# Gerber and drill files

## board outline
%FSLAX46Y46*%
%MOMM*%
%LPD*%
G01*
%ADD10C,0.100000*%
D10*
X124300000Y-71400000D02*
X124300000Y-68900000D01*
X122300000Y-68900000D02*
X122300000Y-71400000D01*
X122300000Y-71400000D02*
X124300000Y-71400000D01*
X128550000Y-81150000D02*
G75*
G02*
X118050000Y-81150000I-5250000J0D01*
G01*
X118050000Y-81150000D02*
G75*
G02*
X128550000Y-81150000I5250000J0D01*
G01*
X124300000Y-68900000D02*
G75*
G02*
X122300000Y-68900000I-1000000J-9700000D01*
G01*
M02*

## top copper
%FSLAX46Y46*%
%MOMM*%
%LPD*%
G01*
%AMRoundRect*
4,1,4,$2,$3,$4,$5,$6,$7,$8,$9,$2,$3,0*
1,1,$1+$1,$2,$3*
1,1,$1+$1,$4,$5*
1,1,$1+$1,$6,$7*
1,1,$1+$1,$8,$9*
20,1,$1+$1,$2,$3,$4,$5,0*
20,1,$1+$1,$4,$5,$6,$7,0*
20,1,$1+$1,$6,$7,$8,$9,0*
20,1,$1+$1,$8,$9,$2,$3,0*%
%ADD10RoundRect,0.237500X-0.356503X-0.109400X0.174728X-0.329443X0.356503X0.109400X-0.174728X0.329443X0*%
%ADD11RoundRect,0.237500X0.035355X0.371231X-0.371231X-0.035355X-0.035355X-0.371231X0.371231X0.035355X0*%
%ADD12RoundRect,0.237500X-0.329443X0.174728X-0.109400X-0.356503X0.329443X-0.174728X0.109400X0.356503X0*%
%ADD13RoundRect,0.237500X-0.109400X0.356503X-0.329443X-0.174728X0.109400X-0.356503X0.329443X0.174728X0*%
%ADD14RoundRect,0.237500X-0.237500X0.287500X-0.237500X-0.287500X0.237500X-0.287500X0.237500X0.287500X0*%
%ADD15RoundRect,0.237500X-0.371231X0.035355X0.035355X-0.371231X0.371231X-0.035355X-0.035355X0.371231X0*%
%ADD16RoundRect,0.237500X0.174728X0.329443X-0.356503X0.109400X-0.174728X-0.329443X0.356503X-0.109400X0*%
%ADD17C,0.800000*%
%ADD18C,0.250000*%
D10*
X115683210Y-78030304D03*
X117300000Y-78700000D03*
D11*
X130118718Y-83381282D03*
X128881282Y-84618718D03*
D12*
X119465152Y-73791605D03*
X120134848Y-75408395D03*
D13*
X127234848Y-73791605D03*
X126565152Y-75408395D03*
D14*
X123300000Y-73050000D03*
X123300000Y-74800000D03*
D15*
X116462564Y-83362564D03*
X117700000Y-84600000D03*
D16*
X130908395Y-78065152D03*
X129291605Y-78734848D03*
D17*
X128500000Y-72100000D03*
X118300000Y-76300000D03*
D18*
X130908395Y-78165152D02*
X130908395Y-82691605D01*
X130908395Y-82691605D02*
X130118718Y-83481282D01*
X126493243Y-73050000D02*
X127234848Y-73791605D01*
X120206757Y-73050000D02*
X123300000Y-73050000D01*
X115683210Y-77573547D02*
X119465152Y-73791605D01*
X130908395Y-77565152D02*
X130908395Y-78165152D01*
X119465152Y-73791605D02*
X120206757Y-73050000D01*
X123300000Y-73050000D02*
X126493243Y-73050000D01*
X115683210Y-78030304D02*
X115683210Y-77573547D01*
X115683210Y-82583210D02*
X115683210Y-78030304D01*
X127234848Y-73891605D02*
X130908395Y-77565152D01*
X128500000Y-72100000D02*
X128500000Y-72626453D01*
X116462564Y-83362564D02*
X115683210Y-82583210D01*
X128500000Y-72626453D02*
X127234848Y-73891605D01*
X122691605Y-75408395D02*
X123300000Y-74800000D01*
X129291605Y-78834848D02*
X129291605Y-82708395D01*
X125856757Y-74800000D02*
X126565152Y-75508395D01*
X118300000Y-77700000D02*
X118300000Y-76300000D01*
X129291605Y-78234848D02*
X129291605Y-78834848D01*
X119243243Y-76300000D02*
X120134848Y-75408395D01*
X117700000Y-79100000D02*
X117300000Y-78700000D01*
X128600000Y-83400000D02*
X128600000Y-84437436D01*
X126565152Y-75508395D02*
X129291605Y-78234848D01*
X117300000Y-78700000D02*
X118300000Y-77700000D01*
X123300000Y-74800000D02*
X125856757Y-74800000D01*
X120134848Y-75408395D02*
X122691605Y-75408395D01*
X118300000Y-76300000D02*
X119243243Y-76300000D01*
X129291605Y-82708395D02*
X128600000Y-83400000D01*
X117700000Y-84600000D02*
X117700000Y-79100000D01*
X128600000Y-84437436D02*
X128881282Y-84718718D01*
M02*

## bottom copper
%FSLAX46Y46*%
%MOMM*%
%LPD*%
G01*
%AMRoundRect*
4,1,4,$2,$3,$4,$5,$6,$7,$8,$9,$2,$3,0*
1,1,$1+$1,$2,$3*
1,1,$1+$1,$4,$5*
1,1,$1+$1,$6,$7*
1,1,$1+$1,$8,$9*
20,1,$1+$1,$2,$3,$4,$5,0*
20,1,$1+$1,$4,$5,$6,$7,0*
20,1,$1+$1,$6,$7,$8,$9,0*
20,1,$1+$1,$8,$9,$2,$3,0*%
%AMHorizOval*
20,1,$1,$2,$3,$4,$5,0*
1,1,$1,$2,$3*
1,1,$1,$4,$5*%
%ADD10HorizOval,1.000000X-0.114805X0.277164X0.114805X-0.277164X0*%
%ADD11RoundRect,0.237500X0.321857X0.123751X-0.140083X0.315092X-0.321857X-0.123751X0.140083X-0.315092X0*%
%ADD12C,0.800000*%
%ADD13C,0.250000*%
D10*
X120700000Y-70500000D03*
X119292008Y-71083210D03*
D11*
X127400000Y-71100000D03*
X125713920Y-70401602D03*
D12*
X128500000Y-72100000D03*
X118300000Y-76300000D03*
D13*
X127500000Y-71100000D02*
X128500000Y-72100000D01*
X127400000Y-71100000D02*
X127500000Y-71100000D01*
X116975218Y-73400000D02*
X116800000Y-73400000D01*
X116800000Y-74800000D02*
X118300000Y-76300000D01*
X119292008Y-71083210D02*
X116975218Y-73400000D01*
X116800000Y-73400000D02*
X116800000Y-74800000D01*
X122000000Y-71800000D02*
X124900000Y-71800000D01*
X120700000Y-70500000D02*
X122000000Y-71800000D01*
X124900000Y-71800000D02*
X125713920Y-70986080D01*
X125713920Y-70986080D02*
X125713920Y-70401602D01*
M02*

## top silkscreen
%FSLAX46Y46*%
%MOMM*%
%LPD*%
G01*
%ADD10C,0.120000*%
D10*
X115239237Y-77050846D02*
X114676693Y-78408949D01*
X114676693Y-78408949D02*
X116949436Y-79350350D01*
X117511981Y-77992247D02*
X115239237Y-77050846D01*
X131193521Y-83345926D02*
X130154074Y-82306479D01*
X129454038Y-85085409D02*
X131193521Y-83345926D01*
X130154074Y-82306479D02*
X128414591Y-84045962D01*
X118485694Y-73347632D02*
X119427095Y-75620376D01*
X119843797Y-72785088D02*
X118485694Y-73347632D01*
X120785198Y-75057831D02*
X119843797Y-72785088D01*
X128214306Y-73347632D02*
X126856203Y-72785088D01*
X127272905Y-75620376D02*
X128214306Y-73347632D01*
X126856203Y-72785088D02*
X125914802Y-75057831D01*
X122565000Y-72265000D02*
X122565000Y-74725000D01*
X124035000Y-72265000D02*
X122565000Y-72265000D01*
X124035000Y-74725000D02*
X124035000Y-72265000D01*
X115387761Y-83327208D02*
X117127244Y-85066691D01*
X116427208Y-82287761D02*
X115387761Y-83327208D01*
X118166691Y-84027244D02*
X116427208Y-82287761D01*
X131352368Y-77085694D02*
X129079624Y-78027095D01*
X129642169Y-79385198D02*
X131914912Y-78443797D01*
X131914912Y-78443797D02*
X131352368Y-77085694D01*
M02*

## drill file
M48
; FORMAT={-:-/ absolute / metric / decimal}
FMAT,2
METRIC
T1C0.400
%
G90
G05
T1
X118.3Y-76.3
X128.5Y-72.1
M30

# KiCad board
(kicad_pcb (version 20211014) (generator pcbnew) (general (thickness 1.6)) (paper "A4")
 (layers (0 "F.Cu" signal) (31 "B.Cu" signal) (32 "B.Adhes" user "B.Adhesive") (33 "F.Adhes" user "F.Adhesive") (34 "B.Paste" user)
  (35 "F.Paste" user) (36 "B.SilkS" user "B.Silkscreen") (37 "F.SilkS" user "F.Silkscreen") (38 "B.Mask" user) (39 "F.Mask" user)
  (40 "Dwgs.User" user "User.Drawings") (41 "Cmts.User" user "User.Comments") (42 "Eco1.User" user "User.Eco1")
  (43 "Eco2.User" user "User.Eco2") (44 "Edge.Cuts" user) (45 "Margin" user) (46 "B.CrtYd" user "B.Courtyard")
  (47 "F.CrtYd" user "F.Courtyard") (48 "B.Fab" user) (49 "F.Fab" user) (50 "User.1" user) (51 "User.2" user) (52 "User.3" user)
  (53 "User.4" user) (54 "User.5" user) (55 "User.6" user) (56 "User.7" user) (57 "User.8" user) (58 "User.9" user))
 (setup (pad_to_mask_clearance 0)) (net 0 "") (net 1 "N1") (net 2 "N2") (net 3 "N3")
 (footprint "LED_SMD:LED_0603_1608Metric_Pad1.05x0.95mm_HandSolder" (layer "F.Cu") (at 116.491605 78.365152 -22.5)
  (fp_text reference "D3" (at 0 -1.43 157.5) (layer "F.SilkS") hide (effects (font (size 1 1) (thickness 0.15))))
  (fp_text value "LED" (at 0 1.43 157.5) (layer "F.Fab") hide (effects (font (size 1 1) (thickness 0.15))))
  (fp_line (start -1.66 -0.735) (end -1.66 0.735) (layer "F.SilkS") (width 0.12))
  (fp_line (start -1.66 0.735) (end 0.8 0.735) (layer "F.SilkS") (width 0.12))
  (fp_line (start 0.8 -0.735) (end -1.66 -0.735) (layer "F.SilkS") (width 0.12))
  (pad "1" smd roundrect (at -0.875 0 337.5) (size 1.05 0.95) (layers "F.Cu" "F.Paste" "F.Mask") (roundrect_rratio 0.25) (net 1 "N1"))
  (pad "2" smd roundrect (at 0.875 0 337.5) (size 1.05 0.95) (layers "F.Cu" "F.Paste" "F.Mask") (roundrect_rratio 0.25) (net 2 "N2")))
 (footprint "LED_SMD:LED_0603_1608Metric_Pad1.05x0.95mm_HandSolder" (layer "F.Cu") (at 129.5 84 -135)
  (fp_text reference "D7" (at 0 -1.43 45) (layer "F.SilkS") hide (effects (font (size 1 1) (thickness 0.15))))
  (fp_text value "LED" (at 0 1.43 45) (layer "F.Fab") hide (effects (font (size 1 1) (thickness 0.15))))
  (fp_line (start -1.66 -0.735) (end -1.66 0.735) (layer "F.SilkS") (width 0.12))
  (fp_line (start 0.8 -0.735) (end -1.66 -0.735) (layer "F.SilkS") (width 0.12))
  (fp_line (start -1.66 0.735) (end 0.8 0.735) (layer "F.SilkS") (width 0.12))
  (pad "1" smd roundrect (at -0.875 0 225) (size 1.05 0.95) (layers "F.Cu" "F.Paste" "F.Mask") (roundrect_rratio 0.25) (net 1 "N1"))
  (pad "2" smd roundrect (at 0.875 0 225) (size 1.05 0.95) (layers "F.Cu" "F.Paste" "F.Mask") (roundrect_rratio 0.25) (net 2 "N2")))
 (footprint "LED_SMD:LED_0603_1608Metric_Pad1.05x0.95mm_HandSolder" (layer "F.Cu") (at 119.8 74.6 -67.5)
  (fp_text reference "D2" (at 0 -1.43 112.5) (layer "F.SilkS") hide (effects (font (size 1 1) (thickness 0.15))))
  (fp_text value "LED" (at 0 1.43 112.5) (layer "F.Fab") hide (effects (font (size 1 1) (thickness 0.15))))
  (fp_line (start -1.66 0.735) (end 0.8 0.735) (layer "F.SilkS") (width 0.12))
  (fp_line (start -1.66 -0.735) (end -1.66 0.735) (layer "F.SilkS") (width 0.12))
  (fp_line (start 0.8 -0.735) (end -1.66 -0.735) (layer "F.SilkS") (width 0.12))
  (pad "1" smd roundrect (at -0.875 0 292.5) (size 1.05 0.95) (layers "F.Cu" "F.Paste" "F.Mask") (roundrect_rratio 0.25) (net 1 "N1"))
  (pad "2" smd roundrect (at 0.875 0 292.5) (size 1.05 0.95) (layers "F.Cu" "F.Paste" "F.Mask") (roundrect_rratio 0.25) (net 2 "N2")))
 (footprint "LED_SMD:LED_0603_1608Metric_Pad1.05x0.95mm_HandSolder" (layer "F.Cu") (at 126.9 74.6 -112.5)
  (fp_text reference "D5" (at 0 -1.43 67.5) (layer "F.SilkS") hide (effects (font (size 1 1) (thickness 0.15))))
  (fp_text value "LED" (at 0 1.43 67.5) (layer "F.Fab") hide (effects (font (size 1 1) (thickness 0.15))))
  (fp_line (start -1.66 -0.735) (end -1.66 0.735) (layer "F.SilkS") (width 0.12))
  (fp_line (start 0.8 -0.735) (end -1.66 -0.735) (layer "F.SilkS") (width 0.12))
  (fp_line (start -1.66 0.735) (end 0.8 0.735) (layer "F.SilkS") (width 0.12))
  (pad "1" smd roundrect (at -0.875 0 247.5) (size 1.05 0.95) (layers "F.Cu" "F.Paste" "F.Mask") (roundrect_rratio 0.25) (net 1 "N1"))
  (pad "2" smd roundrect (at 0.875 0 247.5) (size 1.05 0.95) (layers "F.Cu" "F.Paste" "F.Mask") (roundrect_rratio 0.25) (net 2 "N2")))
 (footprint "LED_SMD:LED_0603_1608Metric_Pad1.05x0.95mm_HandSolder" (layer "F.Cu") (at 123.3 73.925 -90)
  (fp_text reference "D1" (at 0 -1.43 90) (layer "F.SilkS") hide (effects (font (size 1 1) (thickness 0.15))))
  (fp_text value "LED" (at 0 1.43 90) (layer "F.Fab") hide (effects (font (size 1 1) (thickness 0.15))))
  (fp_line (start -1.66 0.735) (end 0.8 0.735) (layer "F.SilkS") (width 0.12))
  (fp_line (start -1.66 -0.735) (end -1.66 0.735) (layer "F.SilkS") (width 0.12))
  (fp_line (start 0.8 -0.735) (end -1.66 -0.735) (layer "F.SilkS") (width 0.12))
  (pad "1" smd roundrect (at -0.875 0 270) (size 1.05 0.95) (layers "F.Cu" "F.Paste" "F.Mask") (roundrect_rratio 0.25) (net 1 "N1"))
  (pad "2" smd roundrect (at 0.875 0 270) (size 1.05 0.95) (layers "F.Cu" "F.Paste" "F.Mask") (roundrect_rratio 0.25) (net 2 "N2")))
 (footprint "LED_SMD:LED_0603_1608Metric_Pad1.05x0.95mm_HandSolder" (layer "F.Cu") (at 117.081282 83.981282 -45)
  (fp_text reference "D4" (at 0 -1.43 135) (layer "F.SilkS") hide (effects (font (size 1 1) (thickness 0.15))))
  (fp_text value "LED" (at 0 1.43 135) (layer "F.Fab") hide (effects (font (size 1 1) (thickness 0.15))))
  (fp_line (start -1.66 0.735) (end 0.8 0.735) (layer "F.SilkS") (width 0.12))
  (fp_line (start -1.66 -0.735) (end -1.66 0.735) (layer "F.SilkS") (width 0.12))
  (fp_line (start 0.8 -0.735) (end -1.66 -0.735) (layer "F.SilkS") (width 0.12))
  (pad "1" smd roundrect (at -0.875 0 315) (size 1.05 0.95) (layers "F.Cu" "F.Paste" "F.Mask") (roundrect_rratio 0.25) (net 1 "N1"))
  (pad "2" smd roundrect (at 0.875 0 315) (size 1.05 0.95) (layers "F.Cu" "F.Paste" "F.Mask") (roundrect_rratio 0.25) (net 2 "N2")))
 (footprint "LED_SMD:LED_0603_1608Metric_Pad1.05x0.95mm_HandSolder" (layer "F.Cu") (at 130.1 78.4 -157.5)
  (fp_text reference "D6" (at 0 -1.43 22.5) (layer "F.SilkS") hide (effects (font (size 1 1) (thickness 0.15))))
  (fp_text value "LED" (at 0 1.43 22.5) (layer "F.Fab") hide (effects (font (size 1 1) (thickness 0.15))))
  (fp_line (start -1.66 0.735) (end 0.8 0.735) (layer "F.SilkS") (width 0.12))
  (fp_line (start 0.8 -0.735) (end -1.66 -0.735) (layer "F.SilkS") (width 0.12))
  (fp_line (start -1.66 -0.735) (end -1.66 0.735) (layer "F.SilkS") (width 0.12))
  (pad "1" smd roundrect (at -0.875 0 202.5) (size 1.05 0.95) (layers "F.Cu" "F.Paste" "F.Mask") (roundrect_rratio 0.25) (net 1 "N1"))
  (pad "2" smd roundrect (at 0.875 0 202.5) (size 1.05 0.95) (layers "F.Cu" "F.Paste" "F.Mask") (roundrect_rratio 0.25) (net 2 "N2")))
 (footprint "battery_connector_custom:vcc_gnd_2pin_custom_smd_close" (layer "B.Cu") (at 119.996004 70.791605 -157.5)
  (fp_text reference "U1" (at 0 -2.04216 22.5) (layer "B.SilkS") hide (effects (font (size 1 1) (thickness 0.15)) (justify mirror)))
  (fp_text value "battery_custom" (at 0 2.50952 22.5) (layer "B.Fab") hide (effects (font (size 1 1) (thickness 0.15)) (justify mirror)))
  (pad "1" smd oval (at -0.762 0 112.5) (size 1.6 1) (layers "B.Cu" "B.Paste" "B.Mask") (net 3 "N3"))
  (pad "2" smd oval (at 0.762 0 112.5) (size 1.6 1) (layers "B.Cu" "B.Paste" "B.Mask") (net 2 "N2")))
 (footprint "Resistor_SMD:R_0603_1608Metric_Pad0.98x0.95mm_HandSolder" (layer "B.Cu") (at 126.55696 70.750801 157.5)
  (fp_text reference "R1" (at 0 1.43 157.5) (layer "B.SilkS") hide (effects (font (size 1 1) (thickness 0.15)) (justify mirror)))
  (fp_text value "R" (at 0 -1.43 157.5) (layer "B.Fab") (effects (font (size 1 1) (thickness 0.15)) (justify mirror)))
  (pad "1" smd roundrect (at -0.9125 0 157.5) (size 0.975 0.95) (layers "B.Cu" "B.Paste" "B.Mask") (roundrect_rratio 0.25) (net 1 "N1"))
  (pad "2" smd roundrect (at 0.9125 0 157.5) (size 0.975 0.95) (layers "B.Cu" "B.Paste" "B.Mask") (roundrect_rratio 0.25) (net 3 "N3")))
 (gr_line (start 124.3 71.4) (end 124.3 68.9) (layer "Edge.Cuts") (width 0.1))
 (gr_line (start 122.3 68.9) (end 122.3 71.4) (layer "Edge.Cuts") (width 0.1))
 (gr_line (start 122.3 71.4) (end 124.3 71.4) (layer "Edge.Cuts") (width 0.1))
 (gr_circle (center 123.3 81.15) (end 128.55 81.15) (layer "Edge.Cuts") (width 0.1) (fill none))
 (gr_arc (start 124.3 68.9) (mid 123.3 88.35141) (end 122.3 68.9) (layer "Edge.Cuts") (width 0.1))
 (segment (start 130.908395 78.165152) (end 130.908395 82.691605) (width 0.25) (layer "F.Cu") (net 1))
 (segment (start 130.908395 82.691605) (end 130.118718 83.481282) (width 0.25) (layer "F.Cu") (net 1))
 (segment (start 126.493243 73.05) (end 127.234848 73.791605) (width 0.25) (layer "F.Cu") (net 1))
 (segment (start 120.206757 73.05) (end 123.3 73.05) (width 0.25) (layer "F.Cu") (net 1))
 (segment (start 115.68321 77.573547) (end 119.465152 73.791605) (width 0.25) (layer "F.Cu") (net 1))
 (segment (start 130.908395 77.565152) (end 130.908395 78.165152) (width 0.25) (layer "F.Cu") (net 1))
 (segment (start 119.465152 73.791605) (end 120.206757 73.05) (width 0.25) (layer "F.Cu") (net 1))
 (segment (start 123.3 73.05) (end 126.493243 73.05) (width 0.25) (layer "F.Cu") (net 1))
 (segment (start 115.68321 78.030304) (end 115.68321 77.573547) (width 0.25) (layer "F.Cu") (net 1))
 (segment (start 115.68321 82.58321) (end 115.68321 78.030304) (width 0.25) (layer "F.Cu") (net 1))
 (segment (start 127.234848 73.891605) (end 130.908395 77.565152) (width 0.25) (layer "F.Cu") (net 1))
 (segment (start 128.5 72.1) (end 128.5 72.626453) (width 0.25) (layer "F.Cu") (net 1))
 (segment (start 116.462564 83.362564) (end 115.68321 82.58321) (width 0.25) (layer "F.Cu") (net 1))
 (segment (start 128.5 72.626453) (end 127.234848 73.891605) (width 0.25) (layer "F.Cu") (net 1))
 (via (at 128.5 72.1) (size 0.8) (drill 0.4) (layers "F.Cu" "B.Cu") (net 1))
 (segment (start 127.5 71.1) (end 128.5 72.1) (width 0.25) (layer "B.Cu") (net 1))
 (segment (start 127.4 71.1) (end 127.5 71.1) (width 0.25) (layer "B.Cu") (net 1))
 (segment (start 122.691605 75.408395) (end 123.3 74.8) (width 0.25) (layer "F.Cu") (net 2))
 (segment (start 129.291605 78.834848) (end 129.291605 82.708395) (width 0.25) (layer "F.Cu") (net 2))
 (segment (start 125.856757 74.8) (end 126.565152 75.508395) (width 0.25) (layer "F.Cu") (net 2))
 (segment (start 118.3 77.7) (end 118.3 76.3) (width 0.25) (layer "F.Cu") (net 2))
 (segment (start 129.291605 78.234848) (end 129.291605 78.834848) (width 0.25) (layer "F.Cu") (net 2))
 (segment (start 119.243243 76.3) (end 120.134848 75.408395) (width 0.25) (layer "F.Cu") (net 2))
 (segment (start 117.7 79.1) (end 117.3 78.7) (width 0.25) (layer "F.Cu") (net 2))
 (segment (start 128.6 83.4) (end 128.6 84.437436) (width 0.25) (layer "F.Cu") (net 2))
 (segment (start 126.565152 75.508395) (end 129.291605 78.234848) (width 0.25) (layer "F.Cu") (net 2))
 (segment (start 117.3 78.7) (end 118.3 77.7) (width 0.25) (layer "F.Cu") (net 2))
 (segment (start 123.3 74.8) (end 125.856757 74.8) (width 0.25) (layer "F.Cu") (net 2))
 (segment (start 120.134848 75.408395) (end 122.691605 75.408395) (width 0.25) (layer "F.Cu") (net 2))
 (segment (start 118.3 76.3) (end 119.243243 76.3) (width 0.25) (layer "F.Cu") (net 2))
 (segment (start 129.291605 82.708395) (end 128.6 83.4) (width 0.25) (layer "F.Cu") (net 2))
 (segment (start 117.7 84.6) (end 117.7 79.1) (width 0.25) (layer "F.Cu") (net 2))
 (segment (start 128.6 84.437436) (end 128.881282 84.718718) (width 0.25) (layer "F.Cu") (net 2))
 (via (at 118.3 76.3) (size 0.8) (drill 0.4) (layers "F.Cu" "B.Cu") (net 2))
 (segment (start 116.975218 73.4) (end 116.8 73.4) (width 0.25) (layer "B.Cu") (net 2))
 (segment (start 116.8 74.8) (end 118.3 76.3) (width 0.25) (layer "B.Cu") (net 2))
 (segment (start 119.292008 71.08321) (end 116.975218 73.4) (width 0.25) (layer "B.Cu") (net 2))
 (segment (start 116.8 73.4) (end 116.8 74.8) (width 0.25) (layer "B.Cu") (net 2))
 (segment (start 122 71.8) (end 124.9 71.8) (width 0.25) (layer "B.Cu") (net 3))
 (segment (start 120.7 70.5) (end 122 71.8) (width 0.25) (layer "B.Cu") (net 3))
 (segment (start 124.9 71.8) (end 125.71392 70.98608) (width 0.25) (layer "B.Cu") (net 3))
 (segment (start 125.71392 70.98608) (end 125.71392 70.401602) (width 0.25) (layer "B.Cu") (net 3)))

